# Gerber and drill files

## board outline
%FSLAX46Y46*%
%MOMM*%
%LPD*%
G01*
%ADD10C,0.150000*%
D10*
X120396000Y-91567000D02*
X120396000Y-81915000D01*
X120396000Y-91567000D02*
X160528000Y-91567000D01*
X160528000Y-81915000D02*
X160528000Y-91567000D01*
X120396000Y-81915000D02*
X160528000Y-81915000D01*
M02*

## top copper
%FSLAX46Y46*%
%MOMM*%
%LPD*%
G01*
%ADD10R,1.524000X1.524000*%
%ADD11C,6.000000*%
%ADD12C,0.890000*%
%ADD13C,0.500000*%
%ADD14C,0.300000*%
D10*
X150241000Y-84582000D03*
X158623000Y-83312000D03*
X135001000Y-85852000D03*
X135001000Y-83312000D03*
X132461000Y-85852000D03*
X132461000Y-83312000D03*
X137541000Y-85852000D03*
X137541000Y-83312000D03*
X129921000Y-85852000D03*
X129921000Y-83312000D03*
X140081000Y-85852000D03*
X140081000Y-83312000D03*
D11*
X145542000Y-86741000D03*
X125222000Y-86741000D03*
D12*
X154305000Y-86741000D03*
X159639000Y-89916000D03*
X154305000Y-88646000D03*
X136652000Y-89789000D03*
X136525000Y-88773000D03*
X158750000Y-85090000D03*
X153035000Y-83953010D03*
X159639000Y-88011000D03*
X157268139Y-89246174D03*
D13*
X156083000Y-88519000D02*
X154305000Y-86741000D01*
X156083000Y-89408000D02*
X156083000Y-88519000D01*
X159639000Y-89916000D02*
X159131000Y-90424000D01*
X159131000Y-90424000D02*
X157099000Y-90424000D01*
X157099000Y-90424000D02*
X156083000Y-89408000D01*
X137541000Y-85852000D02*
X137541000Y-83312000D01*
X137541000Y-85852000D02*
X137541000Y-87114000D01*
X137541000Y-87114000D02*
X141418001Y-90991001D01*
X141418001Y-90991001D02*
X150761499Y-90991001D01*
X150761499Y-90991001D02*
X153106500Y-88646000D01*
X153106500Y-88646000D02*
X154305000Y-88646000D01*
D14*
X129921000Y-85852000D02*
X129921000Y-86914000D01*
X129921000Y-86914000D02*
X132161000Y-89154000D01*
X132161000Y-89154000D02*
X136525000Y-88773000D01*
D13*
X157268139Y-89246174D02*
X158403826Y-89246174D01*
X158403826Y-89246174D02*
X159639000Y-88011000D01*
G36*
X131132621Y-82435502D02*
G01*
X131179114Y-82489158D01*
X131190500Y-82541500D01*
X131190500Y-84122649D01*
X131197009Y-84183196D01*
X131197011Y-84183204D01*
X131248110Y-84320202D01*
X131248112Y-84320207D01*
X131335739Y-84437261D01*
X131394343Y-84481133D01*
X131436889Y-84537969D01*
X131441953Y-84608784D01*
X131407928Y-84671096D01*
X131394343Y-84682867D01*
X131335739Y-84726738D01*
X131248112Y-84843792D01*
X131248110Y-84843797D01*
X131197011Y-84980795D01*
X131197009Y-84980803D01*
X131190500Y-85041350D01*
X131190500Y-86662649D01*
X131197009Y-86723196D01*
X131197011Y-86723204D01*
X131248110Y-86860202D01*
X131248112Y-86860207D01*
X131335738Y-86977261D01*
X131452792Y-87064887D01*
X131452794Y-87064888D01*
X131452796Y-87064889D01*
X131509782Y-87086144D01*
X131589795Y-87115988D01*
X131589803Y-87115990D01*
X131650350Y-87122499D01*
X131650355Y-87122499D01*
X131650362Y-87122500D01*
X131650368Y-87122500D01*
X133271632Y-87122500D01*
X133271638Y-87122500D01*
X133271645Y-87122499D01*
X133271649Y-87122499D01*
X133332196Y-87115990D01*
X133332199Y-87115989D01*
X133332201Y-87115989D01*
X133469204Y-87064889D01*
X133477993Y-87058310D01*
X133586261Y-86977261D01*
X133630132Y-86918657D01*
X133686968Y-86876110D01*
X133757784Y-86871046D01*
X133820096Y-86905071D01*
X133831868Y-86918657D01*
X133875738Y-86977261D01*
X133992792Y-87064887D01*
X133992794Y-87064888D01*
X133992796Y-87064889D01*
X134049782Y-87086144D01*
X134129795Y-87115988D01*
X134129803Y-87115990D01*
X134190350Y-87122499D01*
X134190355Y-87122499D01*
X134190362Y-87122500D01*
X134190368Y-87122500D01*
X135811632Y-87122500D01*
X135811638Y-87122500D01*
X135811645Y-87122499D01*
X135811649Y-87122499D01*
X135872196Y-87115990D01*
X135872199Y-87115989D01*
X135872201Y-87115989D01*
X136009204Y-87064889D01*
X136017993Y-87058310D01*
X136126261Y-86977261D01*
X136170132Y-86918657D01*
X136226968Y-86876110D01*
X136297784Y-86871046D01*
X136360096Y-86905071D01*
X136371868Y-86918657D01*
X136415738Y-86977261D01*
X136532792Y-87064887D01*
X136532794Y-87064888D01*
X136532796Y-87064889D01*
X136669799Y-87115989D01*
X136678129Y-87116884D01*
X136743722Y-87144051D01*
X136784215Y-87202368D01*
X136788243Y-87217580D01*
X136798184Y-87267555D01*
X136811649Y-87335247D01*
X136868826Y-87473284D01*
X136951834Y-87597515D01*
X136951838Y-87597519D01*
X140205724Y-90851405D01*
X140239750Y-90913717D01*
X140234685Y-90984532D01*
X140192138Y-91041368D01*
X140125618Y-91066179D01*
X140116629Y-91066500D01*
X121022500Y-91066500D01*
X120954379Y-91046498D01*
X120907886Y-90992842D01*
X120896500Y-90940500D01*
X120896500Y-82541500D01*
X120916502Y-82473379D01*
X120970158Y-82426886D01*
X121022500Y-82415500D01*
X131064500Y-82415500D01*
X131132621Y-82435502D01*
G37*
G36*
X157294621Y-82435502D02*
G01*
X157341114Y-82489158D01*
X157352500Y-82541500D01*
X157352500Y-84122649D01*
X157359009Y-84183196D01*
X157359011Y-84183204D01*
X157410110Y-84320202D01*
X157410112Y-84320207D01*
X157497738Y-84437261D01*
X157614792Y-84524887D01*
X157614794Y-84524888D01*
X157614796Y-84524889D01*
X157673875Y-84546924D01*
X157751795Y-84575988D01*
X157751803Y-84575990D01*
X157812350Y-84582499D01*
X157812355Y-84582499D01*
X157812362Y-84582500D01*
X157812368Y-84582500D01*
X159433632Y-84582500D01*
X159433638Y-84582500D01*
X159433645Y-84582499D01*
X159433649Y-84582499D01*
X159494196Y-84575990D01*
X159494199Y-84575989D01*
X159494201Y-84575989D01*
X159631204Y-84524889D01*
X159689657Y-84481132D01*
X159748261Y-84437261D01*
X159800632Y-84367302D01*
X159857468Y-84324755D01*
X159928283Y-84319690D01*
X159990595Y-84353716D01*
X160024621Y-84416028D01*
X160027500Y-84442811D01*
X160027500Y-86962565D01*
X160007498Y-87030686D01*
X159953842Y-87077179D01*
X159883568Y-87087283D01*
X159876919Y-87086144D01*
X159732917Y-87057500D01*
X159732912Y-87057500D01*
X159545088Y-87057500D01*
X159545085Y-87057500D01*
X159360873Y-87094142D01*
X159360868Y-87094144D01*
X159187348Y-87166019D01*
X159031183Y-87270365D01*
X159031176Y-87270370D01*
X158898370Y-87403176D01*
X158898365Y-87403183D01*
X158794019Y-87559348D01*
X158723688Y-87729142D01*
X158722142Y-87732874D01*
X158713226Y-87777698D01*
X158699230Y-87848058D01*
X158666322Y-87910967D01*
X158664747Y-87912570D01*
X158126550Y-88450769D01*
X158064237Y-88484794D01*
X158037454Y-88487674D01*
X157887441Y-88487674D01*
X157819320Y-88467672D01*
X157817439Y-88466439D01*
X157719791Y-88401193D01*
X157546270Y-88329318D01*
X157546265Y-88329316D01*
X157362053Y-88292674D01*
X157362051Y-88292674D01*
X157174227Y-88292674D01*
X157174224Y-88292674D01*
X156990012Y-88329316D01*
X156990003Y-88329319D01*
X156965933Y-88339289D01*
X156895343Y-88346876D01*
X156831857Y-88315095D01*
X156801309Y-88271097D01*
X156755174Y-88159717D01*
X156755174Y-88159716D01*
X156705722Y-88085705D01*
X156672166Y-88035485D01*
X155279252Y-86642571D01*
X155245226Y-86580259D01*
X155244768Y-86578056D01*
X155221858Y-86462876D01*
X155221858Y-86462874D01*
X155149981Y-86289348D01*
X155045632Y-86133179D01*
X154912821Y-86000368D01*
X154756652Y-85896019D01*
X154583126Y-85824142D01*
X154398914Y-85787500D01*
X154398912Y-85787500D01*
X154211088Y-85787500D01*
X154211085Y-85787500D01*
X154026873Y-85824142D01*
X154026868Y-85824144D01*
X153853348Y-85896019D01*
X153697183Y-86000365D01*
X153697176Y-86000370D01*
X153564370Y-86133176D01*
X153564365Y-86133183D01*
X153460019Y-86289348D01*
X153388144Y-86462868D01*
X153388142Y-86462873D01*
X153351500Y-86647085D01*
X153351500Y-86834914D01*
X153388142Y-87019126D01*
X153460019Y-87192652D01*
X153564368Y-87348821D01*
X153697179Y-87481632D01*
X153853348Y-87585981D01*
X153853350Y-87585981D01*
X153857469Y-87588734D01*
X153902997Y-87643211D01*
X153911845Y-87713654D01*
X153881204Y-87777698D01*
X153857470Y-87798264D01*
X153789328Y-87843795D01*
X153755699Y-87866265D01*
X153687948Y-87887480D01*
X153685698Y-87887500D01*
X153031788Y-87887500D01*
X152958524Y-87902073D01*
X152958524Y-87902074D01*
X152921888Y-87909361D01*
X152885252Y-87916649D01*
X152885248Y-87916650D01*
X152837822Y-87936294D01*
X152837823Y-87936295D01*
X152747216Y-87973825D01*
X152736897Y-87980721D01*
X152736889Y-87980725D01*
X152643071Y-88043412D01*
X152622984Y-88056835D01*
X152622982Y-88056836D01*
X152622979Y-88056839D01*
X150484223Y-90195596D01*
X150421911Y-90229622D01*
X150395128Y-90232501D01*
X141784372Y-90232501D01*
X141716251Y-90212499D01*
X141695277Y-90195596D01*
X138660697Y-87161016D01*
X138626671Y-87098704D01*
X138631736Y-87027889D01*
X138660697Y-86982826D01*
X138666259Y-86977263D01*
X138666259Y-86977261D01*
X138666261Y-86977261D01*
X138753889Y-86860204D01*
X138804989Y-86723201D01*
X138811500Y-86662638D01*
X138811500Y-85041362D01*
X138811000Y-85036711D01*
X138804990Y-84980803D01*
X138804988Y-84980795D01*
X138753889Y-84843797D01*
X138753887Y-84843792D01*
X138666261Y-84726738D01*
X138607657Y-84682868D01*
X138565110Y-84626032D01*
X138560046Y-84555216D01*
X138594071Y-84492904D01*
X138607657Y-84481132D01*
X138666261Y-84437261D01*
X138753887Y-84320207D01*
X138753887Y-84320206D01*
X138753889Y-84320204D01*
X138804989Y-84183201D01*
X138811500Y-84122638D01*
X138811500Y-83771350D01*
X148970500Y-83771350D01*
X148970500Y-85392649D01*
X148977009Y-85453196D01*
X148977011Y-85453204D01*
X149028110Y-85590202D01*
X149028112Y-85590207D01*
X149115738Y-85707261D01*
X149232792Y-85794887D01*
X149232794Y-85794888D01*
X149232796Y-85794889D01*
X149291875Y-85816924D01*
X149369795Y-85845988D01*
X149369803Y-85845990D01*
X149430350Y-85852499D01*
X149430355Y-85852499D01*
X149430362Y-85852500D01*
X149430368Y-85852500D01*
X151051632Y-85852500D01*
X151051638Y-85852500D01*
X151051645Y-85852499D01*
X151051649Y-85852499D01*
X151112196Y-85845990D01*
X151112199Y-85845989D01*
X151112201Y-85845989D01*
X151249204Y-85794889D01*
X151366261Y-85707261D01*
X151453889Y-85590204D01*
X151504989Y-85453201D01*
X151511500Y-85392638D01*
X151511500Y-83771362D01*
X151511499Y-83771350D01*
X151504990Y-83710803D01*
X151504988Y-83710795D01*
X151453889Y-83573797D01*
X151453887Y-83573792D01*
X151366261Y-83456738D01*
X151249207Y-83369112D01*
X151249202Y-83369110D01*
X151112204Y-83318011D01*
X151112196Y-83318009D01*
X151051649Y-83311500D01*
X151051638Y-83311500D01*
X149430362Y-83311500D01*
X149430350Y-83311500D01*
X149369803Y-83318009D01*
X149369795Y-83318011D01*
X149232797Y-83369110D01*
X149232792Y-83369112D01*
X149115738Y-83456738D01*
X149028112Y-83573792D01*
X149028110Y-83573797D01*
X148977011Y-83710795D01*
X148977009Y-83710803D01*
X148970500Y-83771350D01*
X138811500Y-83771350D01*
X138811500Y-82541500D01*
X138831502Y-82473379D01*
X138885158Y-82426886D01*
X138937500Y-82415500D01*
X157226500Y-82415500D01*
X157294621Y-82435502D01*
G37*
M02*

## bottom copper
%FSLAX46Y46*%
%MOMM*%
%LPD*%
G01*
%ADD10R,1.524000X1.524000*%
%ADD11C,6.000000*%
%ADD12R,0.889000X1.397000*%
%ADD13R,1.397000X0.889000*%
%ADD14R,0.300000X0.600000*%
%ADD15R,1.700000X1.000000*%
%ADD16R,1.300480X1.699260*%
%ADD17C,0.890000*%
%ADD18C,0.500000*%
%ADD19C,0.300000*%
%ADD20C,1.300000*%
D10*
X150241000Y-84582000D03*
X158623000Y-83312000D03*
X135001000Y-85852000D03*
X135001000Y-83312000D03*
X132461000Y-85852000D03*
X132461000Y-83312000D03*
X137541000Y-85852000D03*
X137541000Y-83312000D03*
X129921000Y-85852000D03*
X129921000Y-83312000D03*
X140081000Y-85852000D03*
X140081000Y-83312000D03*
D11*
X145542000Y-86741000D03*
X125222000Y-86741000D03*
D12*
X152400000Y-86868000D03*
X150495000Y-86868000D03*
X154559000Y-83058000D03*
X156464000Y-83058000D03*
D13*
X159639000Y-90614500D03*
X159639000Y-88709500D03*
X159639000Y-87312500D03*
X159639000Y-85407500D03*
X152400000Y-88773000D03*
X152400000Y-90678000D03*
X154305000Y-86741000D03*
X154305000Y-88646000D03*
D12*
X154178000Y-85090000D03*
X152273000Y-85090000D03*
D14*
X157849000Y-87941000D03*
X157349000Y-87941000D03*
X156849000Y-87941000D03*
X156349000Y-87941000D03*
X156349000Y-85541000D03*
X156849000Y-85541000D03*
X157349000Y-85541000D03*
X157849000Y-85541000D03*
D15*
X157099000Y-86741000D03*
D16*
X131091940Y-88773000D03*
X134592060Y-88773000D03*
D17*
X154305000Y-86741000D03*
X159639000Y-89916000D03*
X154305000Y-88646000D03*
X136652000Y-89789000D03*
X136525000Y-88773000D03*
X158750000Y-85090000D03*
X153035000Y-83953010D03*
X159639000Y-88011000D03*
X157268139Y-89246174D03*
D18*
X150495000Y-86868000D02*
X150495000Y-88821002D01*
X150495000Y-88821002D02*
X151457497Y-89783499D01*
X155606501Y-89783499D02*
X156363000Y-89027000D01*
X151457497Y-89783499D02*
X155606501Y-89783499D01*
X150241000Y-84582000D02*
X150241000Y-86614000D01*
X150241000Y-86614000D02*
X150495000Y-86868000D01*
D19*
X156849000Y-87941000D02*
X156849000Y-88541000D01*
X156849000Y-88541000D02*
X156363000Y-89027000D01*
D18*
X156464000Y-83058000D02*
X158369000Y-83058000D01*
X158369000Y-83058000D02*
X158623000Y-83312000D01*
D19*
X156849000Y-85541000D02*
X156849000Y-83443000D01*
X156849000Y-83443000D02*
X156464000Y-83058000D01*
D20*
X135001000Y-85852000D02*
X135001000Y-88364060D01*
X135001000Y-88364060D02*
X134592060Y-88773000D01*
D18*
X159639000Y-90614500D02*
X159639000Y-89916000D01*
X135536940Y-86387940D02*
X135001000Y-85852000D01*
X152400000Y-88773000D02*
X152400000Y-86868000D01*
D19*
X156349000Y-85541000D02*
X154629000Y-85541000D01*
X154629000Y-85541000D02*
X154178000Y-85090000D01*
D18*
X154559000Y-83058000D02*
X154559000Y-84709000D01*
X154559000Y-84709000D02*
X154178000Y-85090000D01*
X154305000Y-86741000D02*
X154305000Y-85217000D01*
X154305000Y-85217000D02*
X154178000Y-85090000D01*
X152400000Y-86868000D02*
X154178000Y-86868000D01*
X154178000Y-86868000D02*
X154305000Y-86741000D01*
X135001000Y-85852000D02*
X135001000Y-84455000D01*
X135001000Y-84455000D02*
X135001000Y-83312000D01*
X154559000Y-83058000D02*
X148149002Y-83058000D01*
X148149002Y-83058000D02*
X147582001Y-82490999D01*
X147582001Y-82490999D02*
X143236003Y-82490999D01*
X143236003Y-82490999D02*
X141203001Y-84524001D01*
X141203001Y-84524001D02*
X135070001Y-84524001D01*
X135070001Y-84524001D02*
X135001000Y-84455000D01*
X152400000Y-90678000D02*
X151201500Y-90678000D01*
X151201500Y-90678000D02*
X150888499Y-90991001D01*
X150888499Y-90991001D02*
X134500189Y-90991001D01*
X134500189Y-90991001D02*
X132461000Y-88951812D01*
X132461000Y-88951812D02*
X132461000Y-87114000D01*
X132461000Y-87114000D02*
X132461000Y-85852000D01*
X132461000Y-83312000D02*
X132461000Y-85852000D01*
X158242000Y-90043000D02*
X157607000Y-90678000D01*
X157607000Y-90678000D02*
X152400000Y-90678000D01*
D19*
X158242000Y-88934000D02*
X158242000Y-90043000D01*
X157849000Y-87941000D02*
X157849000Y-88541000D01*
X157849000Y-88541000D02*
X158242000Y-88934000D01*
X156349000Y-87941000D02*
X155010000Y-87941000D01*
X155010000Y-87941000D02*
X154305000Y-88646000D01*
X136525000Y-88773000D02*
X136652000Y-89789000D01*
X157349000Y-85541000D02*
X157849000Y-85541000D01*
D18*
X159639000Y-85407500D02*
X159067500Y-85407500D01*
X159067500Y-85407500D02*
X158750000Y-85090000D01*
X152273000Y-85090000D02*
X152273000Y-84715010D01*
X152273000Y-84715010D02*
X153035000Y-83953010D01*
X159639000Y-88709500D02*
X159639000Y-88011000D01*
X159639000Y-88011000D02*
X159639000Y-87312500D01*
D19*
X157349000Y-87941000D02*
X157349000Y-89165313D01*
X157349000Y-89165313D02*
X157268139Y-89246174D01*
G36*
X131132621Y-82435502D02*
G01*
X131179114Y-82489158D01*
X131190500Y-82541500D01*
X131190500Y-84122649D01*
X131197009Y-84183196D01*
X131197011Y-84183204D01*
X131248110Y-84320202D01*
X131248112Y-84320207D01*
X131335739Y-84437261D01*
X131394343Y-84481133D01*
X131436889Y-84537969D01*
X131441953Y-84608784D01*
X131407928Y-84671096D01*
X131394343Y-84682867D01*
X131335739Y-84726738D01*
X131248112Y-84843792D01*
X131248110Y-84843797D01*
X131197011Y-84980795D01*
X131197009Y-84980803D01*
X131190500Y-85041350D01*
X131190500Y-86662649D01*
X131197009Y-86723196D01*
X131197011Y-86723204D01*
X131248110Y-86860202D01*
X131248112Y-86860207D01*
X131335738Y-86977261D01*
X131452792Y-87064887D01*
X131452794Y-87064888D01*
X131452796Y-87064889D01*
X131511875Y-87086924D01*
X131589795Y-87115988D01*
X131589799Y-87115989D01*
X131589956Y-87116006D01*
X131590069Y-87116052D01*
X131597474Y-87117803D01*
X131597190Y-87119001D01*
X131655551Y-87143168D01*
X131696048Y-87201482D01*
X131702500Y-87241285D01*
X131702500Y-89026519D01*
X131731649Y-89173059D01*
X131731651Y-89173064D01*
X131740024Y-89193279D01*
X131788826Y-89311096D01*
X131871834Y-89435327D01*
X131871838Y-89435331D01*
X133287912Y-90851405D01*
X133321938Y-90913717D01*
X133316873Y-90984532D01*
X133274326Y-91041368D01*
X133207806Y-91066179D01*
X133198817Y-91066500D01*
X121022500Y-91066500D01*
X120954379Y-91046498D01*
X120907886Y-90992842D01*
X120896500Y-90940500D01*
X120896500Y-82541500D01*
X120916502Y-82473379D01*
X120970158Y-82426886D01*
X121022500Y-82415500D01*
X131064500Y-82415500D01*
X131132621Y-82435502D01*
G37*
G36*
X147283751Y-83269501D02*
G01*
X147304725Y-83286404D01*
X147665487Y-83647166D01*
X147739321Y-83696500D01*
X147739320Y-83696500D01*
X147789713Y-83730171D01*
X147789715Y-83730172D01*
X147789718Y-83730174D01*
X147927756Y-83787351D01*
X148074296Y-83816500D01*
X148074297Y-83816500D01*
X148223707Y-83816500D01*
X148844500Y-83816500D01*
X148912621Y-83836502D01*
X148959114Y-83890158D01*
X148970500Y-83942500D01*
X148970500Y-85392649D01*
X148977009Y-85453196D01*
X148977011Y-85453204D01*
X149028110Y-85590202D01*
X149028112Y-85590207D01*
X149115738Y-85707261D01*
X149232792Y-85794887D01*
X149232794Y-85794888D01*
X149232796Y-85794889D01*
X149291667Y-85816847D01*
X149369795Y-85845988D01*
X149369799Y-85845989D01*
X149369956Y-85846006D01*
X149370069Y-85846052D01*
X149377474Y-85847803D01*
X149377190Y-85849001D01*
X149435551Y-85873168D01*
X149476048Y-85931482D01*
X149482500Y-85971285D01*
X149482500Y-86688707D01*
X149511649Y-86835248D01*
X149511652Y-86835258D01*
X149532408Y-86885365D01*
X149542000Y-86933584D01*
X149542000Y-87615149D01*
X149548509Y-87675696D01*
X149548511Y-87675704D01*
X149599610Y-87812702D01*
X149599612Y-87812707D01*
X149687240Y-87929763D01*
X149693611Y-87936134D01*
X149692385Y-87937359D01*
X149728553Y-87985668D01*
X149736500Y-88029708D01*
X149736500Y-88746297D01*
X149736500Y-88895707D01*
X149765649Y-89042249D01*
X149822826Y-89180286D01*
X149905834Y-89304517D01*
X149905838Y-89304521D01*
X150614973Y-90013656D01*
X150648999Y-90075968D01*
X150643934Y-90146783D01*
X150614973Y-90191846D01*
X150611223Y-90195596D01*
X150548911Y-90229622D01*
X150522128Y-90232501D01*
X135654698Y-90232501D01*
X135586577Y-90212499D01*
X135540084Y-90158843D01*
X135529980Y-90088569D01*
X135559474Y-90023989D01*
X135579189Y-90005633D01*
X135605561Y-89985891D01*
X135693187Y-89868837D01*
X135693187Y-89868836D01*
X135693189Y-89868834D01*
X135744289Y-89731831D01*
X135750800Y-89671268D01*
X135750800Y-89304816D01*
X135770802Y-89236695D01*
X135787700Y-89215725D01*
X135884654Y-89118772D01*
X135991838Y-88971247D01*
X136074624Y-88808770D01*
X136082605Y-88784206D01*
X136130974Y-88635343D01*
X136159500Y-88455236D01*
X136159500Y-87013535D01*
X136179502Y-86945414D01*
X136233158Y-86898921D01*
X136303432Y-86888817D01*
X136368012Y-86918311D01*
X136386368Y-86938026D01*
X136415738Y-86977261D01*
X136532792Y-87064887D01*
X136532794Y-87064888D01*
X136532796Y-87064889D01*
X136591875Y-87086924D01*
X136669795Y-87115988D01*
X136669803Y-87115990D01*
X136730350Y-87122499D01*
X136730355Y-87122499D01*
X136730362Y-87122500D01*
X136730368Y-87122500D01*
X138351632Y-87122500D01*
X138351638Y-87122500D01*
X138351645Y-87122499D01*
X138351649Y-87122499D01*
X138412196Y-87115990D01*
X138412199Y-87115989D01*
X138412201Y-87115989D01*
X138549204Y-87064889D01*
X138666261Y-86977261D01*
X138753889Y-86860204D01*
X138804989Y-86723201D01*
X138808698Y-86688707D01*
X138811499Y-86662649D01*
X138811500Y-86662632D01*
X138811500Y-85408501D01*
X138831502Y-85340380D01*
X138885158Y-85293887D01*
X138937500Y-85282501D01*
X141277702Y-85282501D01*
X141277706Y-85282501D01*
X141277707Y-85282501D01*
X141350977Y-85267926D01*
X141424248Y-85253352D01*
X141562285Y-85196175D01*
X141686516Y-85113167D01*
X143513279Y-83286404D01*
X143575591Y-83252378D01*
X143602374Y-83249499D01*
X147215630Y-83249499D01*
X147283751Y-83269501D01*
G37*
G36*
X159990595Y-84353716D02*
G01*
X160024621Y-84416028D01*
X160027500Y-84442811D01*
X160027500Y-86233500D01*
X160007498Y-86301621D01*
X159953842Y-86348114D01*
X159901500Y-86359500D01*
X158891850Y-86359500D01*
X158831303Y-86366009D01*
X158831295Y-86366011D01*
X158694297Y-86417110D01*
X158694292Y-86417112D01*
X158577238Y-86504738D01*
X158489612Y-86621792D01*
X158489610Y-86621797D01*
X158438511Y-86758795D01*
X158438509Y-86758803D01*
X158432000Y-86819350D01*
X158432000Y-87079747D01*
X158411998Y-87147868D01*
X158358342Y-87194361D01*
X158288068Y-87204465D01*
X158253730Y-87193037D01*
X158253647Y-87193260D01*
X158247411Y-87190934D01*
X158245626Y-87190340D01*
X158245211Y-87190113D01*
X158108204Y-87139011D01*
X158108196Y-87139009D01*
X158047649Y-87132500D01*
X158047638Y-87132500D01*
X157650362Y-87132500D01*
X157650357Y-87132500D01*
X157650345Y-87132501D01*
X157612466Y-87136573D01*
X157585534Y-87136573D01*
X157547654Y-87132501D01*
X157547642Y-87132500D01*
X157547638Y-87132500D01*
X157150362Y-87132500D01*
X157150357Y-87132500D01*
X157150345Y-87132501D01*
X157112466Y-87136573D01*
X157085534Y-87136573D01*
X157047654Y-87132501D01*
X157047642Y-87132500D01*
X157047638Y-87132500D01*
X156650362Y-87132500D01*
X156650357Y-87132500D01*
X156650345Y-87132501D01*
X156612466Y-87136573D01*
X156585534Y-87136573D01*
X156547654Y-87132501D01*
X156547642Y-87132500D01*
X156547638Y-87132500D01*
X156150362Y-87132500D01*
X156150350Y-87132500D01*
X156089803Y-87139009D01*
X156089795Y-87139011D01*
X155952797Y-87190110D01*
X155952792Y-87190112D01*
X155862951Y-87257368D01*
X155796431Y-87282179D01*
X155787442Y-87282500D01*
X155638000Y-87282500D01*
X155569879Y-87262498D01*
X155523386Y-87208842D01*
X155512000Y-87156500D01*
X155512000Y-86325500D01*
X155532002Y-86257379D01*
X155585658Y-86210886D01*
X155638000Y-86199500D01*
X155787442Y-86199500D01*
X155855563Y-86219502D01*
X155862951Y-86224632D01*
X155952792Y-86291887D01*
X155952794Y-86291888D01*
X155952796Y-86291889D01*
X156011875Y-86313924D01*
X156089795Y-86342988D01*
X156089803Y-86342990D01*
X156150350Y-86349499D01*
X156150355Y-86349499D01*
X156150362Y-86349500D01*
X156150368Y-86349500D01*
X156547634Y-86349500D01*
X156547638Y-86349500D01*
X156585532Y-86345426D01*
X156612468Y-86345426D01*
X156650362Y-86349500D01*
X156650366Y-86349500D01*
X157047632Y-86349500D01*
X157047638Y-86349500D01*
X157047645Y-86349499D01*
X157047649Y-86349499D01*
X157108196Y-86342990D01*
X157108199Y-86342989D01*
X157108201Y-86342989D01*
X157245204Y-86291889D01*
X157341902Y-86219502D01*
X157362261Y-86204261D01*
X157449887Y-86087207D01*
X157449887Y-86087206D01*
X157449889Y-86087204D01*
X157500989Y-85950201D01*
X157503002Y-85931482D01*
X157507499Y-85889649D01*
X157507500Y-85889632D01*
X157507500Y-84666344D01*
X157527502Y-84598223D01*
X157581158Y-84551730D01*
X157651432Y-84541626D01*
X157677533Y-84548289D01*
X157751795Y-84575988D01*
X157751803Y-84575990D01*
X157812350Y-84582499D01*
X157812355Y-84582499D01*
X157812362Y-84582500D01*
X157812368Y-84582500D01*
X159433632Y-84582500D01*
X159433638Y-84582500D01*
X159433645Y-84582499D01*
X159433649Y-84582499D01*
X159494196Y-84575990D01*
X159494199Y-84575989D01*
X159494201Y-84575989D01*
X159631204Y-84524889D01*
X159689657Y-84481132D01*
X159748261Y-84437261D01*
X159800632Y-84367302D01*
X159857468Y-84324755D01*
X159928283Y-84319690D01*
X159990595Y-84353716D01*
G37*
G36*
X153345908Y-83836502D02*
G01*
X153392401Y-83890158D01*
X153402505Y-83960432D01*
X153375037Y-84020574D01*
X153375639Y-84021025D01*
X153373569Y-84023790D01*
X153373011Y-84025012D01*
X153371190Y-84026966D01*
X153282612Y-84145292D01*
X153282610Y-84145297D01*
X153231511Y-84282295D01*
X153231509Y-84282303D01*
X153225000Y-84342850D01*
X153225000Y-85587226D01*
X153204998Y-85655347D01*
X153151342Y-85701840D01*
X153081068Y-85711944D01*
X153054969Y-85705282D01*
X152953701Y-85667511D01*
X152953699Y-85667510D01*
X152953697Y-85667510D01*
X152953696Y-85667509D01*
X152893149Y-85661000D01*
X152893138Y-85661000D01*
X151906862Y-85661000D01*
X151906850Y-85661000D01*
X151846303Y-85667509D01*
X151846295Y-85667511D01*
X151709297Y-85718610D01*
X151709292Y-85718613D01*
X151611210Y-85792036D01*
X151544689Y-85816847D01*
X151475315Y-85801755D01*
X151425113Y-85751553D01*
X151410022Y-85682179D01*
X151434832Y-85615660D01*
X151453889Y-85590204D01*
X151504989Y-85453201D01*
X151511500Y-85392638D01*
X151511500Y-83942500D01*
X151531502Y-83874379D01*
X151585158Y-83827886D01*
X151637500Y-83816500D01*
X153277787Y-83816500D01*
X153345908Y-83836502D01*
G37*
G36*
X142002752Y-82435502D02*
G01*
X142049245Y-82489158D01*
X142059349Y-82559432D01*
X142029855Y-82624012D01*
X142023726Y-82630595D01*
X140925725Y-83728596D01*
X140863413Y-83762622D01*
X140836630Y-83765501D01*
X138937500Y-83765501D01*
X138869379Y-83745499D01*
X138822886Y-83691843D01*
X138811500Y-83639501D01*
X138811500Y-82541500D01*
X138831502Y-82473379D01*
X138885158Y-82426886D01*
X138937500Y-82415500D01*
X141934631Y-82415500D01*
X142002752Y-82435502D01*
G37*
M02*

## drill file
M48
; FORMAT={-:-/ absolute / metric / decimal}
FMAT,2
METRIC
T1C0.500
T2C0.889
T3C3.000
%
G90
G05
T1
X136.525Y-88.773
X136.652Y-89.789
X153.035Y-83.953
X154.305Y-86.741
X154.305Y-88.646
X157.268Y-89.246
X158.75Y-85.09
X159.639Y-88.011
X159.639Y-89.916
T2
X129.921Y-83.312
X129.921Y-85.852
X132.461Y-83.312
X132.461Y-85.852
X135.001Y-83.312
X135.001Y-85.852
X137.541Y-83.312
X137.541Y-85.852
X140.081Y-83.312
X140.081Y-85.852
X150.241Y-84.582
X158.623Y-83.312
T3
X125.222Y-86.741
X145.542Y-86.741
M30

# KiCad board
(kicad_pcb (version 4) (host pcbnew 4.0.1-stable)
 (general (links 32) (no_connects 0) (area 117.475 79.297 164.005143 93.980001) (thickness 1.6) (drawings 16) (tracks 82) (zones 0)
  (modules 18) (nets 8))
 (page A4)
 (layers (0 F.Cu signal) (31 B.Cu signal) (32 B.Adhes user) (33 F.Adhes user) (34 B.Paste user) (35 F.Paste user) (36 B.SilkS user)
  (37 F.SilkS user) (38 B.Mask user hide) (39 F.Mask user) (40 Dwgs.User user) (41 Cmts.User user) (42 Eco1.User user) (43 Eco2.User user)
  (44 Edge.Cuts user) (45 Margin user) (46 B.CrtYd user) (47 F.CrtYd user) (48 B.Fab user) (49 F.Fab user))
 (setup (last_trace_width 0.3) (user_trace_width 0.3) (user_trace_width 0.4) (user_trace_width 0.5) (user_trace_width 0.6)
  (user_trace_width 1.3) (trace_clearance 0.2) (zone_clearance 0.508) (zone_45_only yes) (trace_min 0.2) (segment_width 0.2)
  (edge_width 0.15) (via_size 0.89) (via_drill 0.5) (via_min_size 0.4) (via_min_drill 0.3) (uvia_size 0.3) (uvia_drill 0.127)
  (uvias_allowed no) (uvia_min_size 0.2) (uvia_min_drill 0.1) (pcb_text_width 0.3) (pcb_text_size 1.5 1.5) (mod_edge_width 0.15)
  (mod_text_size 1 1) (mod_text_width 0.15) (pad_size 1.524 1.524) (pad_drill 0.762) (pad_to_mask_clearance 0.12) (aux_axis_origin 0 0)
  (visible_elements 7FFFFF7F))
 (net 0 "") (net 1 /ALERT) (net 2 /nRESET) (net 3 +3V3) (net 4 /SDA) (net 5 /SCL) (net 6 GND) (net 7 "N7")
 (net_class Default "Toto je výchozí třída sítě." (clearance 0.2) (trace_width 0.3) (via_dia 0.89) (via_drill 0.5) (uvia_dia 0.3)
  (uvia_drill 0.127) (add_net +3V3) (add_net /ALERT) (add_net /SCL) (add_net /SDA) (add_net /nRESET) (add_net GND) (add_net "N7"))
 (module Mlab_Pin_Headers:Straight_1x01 (layer F.Cu) (at 150.241 84.582)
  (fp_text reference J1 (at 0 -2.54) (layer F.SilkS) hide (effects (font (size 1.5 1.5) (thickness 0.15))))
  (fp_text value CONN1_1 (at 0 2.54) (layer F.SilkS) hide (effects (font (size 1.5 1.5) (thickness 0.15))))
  (pad 1 thru_hole rect (at 0 0) (size 1.524 1.524) (drill 0.889) (layers *.Cu *.Mask F.SilkS) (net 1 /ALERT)))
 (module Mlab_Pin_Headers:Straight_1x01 (layer F.Cu) (at 158.623 83.312)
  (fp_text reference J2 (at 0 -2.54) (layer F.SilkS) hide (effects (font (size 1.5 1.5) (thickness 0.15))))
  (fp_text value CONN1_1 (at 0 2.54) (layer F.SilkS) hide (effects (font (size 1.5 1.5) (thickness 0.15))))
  (pad 1 thru_hole rect (at 0 0) (size 1.524 1.524) (drill 0.889) (layers *.Cu *.Mask F.SilkS) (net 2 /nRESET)))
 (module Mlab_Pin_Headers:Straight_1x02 (layer F.Cu) (at 135.001 84.582)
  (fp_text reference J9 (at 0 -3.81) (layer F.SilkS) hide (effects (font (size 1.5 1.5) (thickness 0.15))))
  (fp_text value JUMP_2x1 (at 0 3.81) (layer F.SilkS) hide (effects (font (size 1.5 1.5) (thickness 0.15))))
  (pad 2 thru_hole rect (at 0 1.27) (size 1.524 1.524) (drill 0.889) (layers *.Cu *.Mask F.SilkS) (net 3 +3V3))
  (pad 1 thru_hole rect (at 0 -1.27) (size 1.524 1.524) (drill 0.889) (layers *.Cu *.Mask F.SilkS) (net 3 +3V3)))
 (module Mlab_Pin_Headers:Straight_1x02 (layer F.Cu) (at 132.461 84.582)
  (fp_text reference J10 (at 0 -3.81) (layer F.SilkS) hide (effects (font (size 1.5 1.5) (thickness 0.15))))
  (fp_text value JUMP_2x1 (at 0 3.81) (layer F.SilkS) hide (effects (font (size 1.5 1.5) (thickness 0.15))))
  (pad 2 thru_hole rect (at 0 1.27) (size 1.524 1.524) (drill 0.889) (layers *.Cu *.Mask F.SilkS) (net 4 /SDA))
  (pad 1 thru_hole rect (at 0 -1.27) (size 1.524 1.524) (drill 0.889) (layers *.Cu *.Mask F.SilkS) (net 4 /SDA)))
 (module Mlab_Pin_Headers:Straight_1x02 (layer F.Cu) (at 137.541 84.582)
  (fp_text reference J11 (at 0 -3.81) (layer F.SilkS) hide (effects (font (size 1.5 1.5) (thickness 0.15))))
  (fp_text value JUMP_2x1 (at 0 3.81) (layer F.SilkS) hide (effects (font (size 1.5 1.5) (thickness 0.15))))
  (pad 2 thru_hole rect (at 0 1.27) (size 1.524 1.524) (drill 0.889) (layers *.Cu *.Mask F.SilkS) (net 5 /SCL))
  (pad 1 thru_hole rect (at 0 -1.27) (size 1.524 1.524) (drill 0.889) (layers *.Cu *.Mask F.SilkS) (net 5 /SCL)))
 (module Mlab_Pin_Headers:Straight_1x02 (layer F.Cu) (at 129.921 84.582)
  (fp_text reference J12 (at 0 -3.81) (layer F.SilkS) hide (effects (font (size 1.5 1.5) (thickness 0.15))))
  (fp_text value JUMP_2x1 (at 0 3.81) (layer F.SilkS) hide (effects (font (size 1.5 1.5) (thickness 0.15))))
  (pad 2 thru_hole rect (at 0 1.27) (size 1.524 1.524) (drill 0.889) (layers *.Cu *.Mask F.SilkS) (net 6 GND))
  (pad 1 thru_hole rect (at 0 -1.27) (size 1.524 1.524) (drill 0.889) (layers *.Cu *.Mask F.SilkS) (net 6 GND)))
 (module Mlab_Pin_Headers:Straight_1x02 (layer F.Cu) (at 140.081 84.582)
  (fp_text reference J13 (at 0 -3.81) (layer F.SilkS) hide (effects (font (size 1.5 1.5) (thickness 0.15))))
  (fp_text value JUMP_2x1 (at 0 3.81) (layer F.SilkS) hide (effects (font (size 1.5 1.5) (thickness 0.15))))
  (pad 2 thru_hole rect (at 0 1.27) (size 1.524 1.524) (drill 0.889) (layers *.Cu *.Mask F.SilkS) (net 6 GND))
  (pad 1 thru_hole rect (at 0 -1.27) (size 1.524 1.524) (drill 0.889) (layers *.Cu *.Mask F.SilkS) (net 6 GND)))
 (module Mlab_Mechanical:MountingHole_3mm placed (layer F.Cu) (at 145.542 86.741)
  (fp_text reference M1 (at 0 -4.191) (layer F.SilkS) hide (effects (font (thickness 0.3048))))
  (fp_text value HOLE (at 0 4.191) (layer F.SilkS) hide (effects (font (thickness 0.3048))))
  (pad 1 thru_hole circle (at 0 0) (size 6 6) (drill 3) (layers *.Cu *.Adhes *.Mask) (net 6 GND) (clearance 1) (zone_connect 2)))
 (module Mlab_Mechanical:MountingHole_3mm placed (layer F.Cu) (at 125.222 86.741)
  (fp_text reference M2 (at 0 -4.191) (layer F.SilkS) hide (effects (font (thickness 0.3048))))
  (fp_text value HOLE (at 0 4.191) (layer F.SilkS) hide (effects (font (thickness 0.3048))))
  (pad 1 thru_hole circle (at 0 0) (size 6 6) (drill 3) (layers *.Cu *.Adhes *.Mask) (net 6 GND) (clearance 1) (zone_connect 2)))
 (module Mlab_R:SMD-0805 (layer B.Cu) (at 151.4475 86.868 180)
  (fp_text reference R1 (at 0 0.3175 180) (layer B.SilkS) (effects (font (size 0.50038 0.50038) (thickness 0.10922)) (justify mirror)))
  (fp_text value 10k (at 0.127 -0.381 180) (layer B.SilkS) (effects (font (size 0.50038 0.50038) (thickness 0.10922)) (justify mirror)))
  (pad 1 smd rect (at -0.9525 0 180) (size 0.889 1.397) (layers B.Cu B.Paste B.Mask) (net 3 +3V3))
  (pad 2 smd rect (at 0.9525 0 180) (size 0.889 1.397) (layers B.Cu B.Paste B.Mask) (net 1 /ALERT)))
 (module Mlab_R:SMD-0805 (layer B.Cu) (at 155.5115 83.058)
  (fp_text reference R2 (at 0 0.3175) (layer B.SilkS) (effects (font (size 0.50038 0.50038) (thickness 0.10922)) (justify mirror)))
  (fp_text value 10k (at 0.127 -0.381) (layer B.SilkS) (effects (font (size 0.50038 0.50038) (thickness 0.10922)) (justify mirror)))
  (pad 1 smd rect (at -0.9525 0) (size 0.889 1.397) (layers B.Cu B.Paste B.Mask) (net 3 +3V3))
  (pad 2 smd rect (at 0.9525 0) (size 0.889 1.397) (layers B.Cu B.Paste B.Mask) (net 2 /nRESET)))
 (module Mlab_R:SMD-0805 (layer B.Cu) (at 159.639 89.662 90)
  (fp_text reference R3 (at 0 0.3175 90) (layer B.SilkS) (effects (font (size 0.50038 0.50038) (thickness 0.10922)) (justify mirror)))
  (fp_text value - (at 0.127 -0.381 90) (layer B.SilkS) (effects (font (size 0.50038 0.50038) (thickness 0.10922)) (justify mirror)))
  (pad 1 smd rect (at -0.9525 0 90) (size 0.889 1.397) (layers B.Cu B.Paste B.Mask) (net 3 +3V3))
  (pad 2 smd rect (at 0.9525 0 90) (size 0.889 1.397) (layers B.Cu B.Paste B.Mask) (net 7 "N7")))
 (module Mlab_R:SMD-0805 (layer B.Cu) (at 159.639 86.36 90)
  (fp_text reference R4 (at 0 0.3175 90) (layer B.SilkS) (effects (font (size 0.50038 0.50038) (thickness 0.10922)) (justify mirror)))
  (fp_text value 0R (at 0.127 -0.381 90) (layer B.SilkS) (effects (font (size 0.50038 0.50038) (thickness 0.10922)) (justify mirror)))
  (pad 1 smd rect (at -0.9525 0 90) (size 0.889 1.397) (layers B.Cu B.Paste B.Mask) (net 7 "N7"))
  (pad 2 smd rect (at 0.9525 0 90) (size 0.889 1.397) (layers B.Cu B.Paste B.Mask) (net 6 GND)))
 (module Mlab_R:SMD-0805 (layer B.Cu) (at 152.4 89.7255 270)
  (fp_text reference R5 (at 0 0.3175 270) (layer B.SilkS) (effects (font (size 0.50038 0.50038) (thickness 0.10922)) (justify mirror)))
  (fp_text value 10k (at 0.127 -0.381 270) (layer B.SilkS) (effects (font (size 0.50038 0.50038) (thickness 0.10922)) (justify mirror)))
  (pad 1 smd rect (at -0.9525 0 270) (size 0.889 1.397) (layers B.Cu B.Paste B.Mask) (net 3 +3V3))
  (pad 2 smd rect (at 0.9525 0 270) (size 0.889 1.397) (layers B.Cu B.Paste B.Mask) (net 4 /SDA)))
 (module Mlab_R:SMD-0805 (layer B.Cu) (at 154.305 87.6935 270)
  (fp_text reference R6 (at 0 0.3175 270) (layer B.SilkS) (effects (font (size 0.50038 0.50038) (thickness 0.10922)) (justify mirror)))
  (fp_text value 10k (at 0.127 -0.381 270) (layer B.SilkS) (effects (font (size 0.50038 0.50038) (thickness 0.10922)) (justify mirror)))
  (pad 1 smd rect (at -0.9525 0 270) (size 0.889 1.397) (layers B.Cu B.Paste B.Mask) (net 3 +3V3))
  (pad 2 smd rect (at 0.9525 0 270) (size 0.889 1.397) (layers B.Cu B.Paste B.Mask) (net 5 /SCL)))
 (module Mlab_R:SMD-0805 (layer B.Cu) (at 153.2255 85.09 180)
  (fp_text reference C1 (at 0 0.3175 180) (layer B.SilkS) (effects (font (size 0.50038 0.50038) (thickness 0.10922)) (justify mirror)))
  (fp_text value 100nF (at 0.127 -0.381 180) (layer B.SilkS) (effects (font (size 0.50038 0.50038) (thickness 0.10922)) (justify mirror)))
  (pad 1 smd rect (at -0.9525 0 180) (size 0.889 1.397) (layers B.Cu B.Paste B.Mask) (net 3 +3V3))
  (pad 2 smd rect (at 0.9525 0 180) (size 0.889 1.397) (layers B.Cu B.Paste B.Mask) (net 6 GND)))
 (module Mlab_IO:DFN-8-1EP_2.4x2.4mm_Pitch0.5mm (layer B.Cu) (at 157.099 86.741 90)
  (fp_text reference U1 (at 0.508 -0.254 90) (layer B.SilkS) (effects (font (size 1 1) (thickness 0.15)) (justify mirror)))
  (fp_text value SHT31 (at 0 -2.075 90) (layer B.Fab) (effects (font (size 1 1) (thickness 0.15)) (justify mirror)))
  (pad 1 smd rect (at -1.2 0.75 90) (size 0.6 0.3) (layers B.Cu B.Paste B.Mask) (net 4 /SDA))
  (pad 2 smd rect (at -1.2 0.25 90) (size 0.6 0.3) (layers B.Cu B.Paste B.Mask) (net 7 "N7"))
  (pad 3 smd rect (at -1.2 -0.25 90) (size 0.6 0.3) (layers B.Cu B.Paste B.Mask) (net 1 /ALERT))
  (pad 4 smd rect (at -1.2 -0.75 90) (size 0.6 0.3) (layers B.Cu B.Paste B.Mask) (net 5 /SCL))
  (pad 5 smd rect (at 1.2 -0.75 90) (size 0.6 0.3) (layers B.Cu B.Paste B.Mask) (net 3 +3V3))
  (pad 6 smd rect (at 1.2 -0.25 90) (size 0.6 0.3) (layers B.Cu B.Paste B.Mask) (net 2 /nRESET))
  (pad 7 smd rect (at 1.2 0.25 90) (size 0.6 0.3) (layers B.Cu B.Paste B.Mask) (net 6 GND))
  (pad 8 smd rect (at 1.2 0.75 90) (size 0.6 0.3) (layers B.Cu B.Paste B.Mask) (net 6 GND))
  (pad 9 smd rect (at 0 0 90) (size 1 1.7) (layers B.Cu B.Paste B.Mask) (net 6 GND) (solder_paste_margin_ratio -0.2)))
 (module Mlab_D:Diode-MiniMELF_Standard (layer B.Cu) (at 132.842 88.773)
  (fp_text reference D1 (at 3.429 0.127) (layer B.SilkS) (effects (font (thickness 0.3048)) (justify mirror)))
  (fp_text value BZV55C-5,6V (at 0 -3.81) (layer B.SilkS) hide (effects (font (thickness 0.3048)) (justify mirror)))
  (pad 1 smd rect (at -1.75006 0) (size 1.30048 1.69926) (layers B.Cu B.Paste B.Mask) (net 6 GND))
  (pad 2 smd rect (at 1.75006 0) (size 1.30048 1.69926) (layers B.Cu B.Paste B.Mask) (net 3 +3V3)))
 (gr_line (start 120.396 91.567) (end 120.396 81.915) (angle 90) (layer Edge.Cuts) (width 0.15))
 (gr_line (start 120.396 91.567) (end 160.528 91.567) (angle 90) (layer Edge.Cuts) (width 0.15))
 (gr_line (start 160.528 81.915) (end 160.528 91.567) (angle 90) (layer Edge.Cuts) (width 0.15))
 (gr_line (start 120.396 81.915) (end 160.528 81.915) (angle 90) (layer Edge.Cuts) (width 0.15))
 (segment (start 150.495 86.868) (end 150.495 88.821002) (width 0.5) (layer B.Cu) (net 1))
 (segment (start 150.495 88.821002) (end 151.457497 89.783499) (width 0.5) (layer B.Cu) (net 1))
 (segment (start 155.606501 89.783499) (end 156.363 89.027) (width 0.5) (layer B.Cu) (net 1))
 (segment (start 151.457497 89.783499) (end 155.606501 89.783499) (width 0.5) (layer B.Cu) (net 1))
 (segment (start 150.241 84.582) (end 150.241 86.614) (width 0.5) (layer B.Cu) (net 1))
 (segment (start 150.241 86.614) (end 150.495 86.868) (width 0.5) (layer B.Cu) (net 1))
 (segment (start 156.849 87.941) (end 156.849 88.541) (width 0.3) (layer B.Cu) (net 1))
 (segment (start 156.849 88.541) (end 156.363 89.027) (width 0.3) (layer B.Cu) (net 1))
 (segment (start 156.464 83.058) (end 158.369 83.058) (width 0.5) (layer B.Cu) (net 2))
 (segment (start 158.369 83.058) (end 158.623 83.312) (width 0.5) (layer B.Cu) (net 2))
 (segment (start 156.849 85.541) (end 156.849 83.443) (width 0.3) (layer B.Cu) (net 2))
 (segment (start 156.849 83.443) (end 156.464 83.058) (width 0.3) (layer B.Cu) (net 2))
 (segment (start 135.001 85.852) (end 135.001 88.36406) (width 1.3) (layer B.Cu) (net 3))
 (segment (start 135.001 88.36406) (end 134.59206 88.773) (width 1.3) (layer B.Cu) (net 3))
 (segment (start 156.083 88.519) (end 154.305 86.741) (width 0.5) (layer F.Cu) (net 3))
 (segment (start 156.083 89.408) (end 156.083 88.519) (width 0.5) (layer F.Cu) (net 3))
 (segment (start 159.639 89.916) (end 159.131 90.424) (width 0.5) (layer F.Cu) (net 3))
 (segment (start 159.131 90.424) (end 157.099 90.424) (width 0.5) (layer F.Cu) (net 3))
 (segment (start 157.099 90.424) (end 156.083 89.408) (width 0.5) (layer F.Cu) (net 3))
 (via (at 154.305 86.741) (size 0.89) (drill 0.5) (layers F.Cu B.Cu) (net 3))
 (segment (start 159.639 90.6145) (end 159.639 89.916) (width 0.5) (layer B.Cu) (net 3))
 (via (at 159.639 89.916) (size 0.89) (drill 0.5) (layers F.Cu B.Cu) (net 3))
 (segment (start 135.53694 86.38794) (end 135.001 85.852) (width 0.5) (layer B.Cu) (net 3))
 (segment (start 152.4 88.773) (end 152.4 86.868) (width 0.5) (layer B.Cu) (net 3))
 (segment (start 156.349 85.541) (end 154.629 85.541) (width 0.3) (layer B.Cu) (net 3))
 (segment (start 154.629 85.541) (end 154.178 85.09) (width 0.3) (layer B.Cu) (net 3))
 (segment (start 154.559 83.058) (end 154.559 84.709) (width 0.5) (layer B.Cu) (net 3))
 (segment (start 154.559 84.709) (end 154.178 85.09) (width 0.5) (layer B.Cu) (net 3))
 (segment (start 154.305 86.741) (end 154.305 85.217) (width 0.5) (layer B.Cu) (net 3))
 (segment (start 154.305 85.217) (end 154.178 85.09) (width 0.5) (layer B.Cu) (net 3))
 (segment (start 152.4 86.868) (end 154.178 86.868) (width 0.5) (layer B.Cu) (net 3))
 (segment (start 154.178 86.868) (end 154.305 86.741) (width 0.5) (layer B.Cu) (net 3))
 (segment (start 135.001 85.852) (end 135.001 84.455) (width 0.5) (layer B.Cu) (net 3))
 (segment (start 135.001 84.455) (end 135.001 83.312) (width 0.5) (layer B.Cu) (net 3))
 (segment (start 154.559 83.058) (end 148.149002 83.058) (width 0.5) (layer B.Cu) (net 3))
 (segment (start 148.149002 83.058) (end 147.582001 82.490999) (width 0.5) (layer B.Cu) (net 3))
 (segment (start 147.582001 82.490999) (end 143.236003 82.490999) (width 0.5) (layer B.Cu) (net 3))
 (segment (start 143.236003 82.490999) (end 141.203001 84.524001) (width 0.5) (layer B.Cu) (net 3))
 (segment (start 141.203001 84.524001) (end 135.070001 84.524001) (width 0.5) (layer B.Cu) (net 3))
 (segment (start 135.070001 84.524001) (end 135.001 84.455) (width 0.5) (layer B.Cu) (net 3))
 (segment (start 152.4 90.678) (end 151.2015 90.678) (width 0.5) (layer B.Cu) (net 4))
 (segment (start 151.2015 90.678) (end 150.888499 90.991001) (width 0.5) (layer B.Cu) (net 4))
 (segment (start 150.888499 90.991001) (end 134.500189 90.991001) (width 0.5) (layer B.Cu) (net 4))
 (segment (start 134.500189 90.991001) (end 132.461 88.951812) (width 0.5) (layer B.Cu) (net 4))
 (segment (start 132.461 88.951812) (end 132.461 87.114) (width 0.5) (layer B.Cu) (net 4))
 (segment (start 132.461 87.114) (end 132.461 85.852) (width 0.5) (layer B.Cu) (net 4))
 (segment (start 132.461 83.312) (end 132.461 85.852) (width 0.5) (layer B.Cu) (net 4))
 (segment (start 158.242 90.043) (end 157.607 90.678) (width 0.5) (layer B.Cu) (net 4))
 (segment (start 157.607 90.678) (end 152.4 90.678) (width 0.5) (layer B.Cu) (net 4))
 (segment (start 158.242 88.934) (end 158.242 90.043) (width 0.3) (layer B.Cu) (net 4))
 (segment (start 157.849 87.941) (end 157.849 88.541) (width 0.3) (layer B.Cu) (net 4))
 (segment (start 157.849 88.541) (end 158.242 88.934) (width 0.3) (layer B.Cu) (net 4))
 (segment (start 137.541 85.852) (end 137.541 83.312) (width 0.5) (layer F.Cu) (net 5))
 (segment (start 137.541 85.852) (end 137.541 87.114) (width 0.5) (layer F.Cu) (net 5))
 (segment (start 137.541 87.114) (end 141.418001 90.991001) (width 0.5) (layer F.Cu) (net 5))
 (segment (start 141.418001 90.991001) (end 150.761499 90.991001) (width 0.5) (layer F.Cu) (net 5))
 (segment (start 150.761499 90.991001) (end 153.1065 88.646) (width 0.5) (layer F.Cu) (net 5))
 (segment (start 153.1065 88.646) (end 154.305 88.646) (width 0.5) (layer F.Cu) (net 5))
 (via (at 154.305 88.646) (size 0.89) (drill 0.5) (layers F.Cu B.Cu) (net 5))
 (segment (start 156.349 87.941) (end 155.01 87.941) (width 0.3) (layer B.Cu) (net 5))
 (segment (start 155.01 87.941) (end 154.305 88.646) (width 0.3) (layer B.Cu) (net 5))
 (segment (start 136.525 88.773) (end 136.652 89.789) (width 0.3) (layer B.Cu) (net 6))
 (via (at 136.652 89.789) (size 0.89) (drill 0.5) (layers F.Cu B.Cu) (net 6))
 (segment (start 129.921 85.852) (end 129.921 86.914) (width 0.3) (layer F.Cu) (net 6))
 (segment (start 129.921 86.914) (end 132.161 89.154) (width 0.3) (layer F.Cu) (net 6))
 (segment (start 132.161 89.154) (end 136.525 88.773) (width 0.3) (layer F.Cu) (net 6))
 (via (at 136.525 88.773) (size 0.89) (drill 0.5) (layers F.Cu B.Cu) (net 6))
 (segment (start 157.349 85.541) (end 157.849 85.541) (width 0.3) (layer B.Cu) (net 6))
 (segment (start 159.639 85.4075) (end 159.0675 85.4075) (width 0.5) (layer B.Cu) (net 6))
 (segment (start 159.0675 85.4075) (end 158.75 85.09) (width 0.5) (layer B.Cu) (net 6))
 (via (at 158.75 85.09) (size 0.89) (drill 0.5) (layers F.Cu B.Cu) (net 6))
 (segment (start 152.273 85.09) (end 152.273 84.71501) (width 0.5) (layer B.Cu) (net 6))
 (segment (start 152.273 84.71501) (end 153.035 83.95301) (width 0.5) (layer B.Cu) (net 6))
 (via (at 153.035 83.95301) (size 0.89) (drill 0.5) (layers F.Cu B.Cu) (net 6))
 (segment (start 159.639 88.7095) (end 159.639 88.011) (width 0.5) (layer B.Cu) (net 7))
 (segment (start 159.639 88.011) (end 159.639 87.3125) (width 0.5) (layer B.Cu) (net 7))
 (segment (start 157.268139 89.246174) (end 158.403826 89.246174) (width 0.5) (layer F.Cu) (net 7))
 (segment (start 158.403826 89.246174) (end 159.639 88.011) (width 0.5) (layer F.Cu) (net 7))
 (via (at 159.639 88.011) (size 0.89) (drill 0.5) (layers F.Cu B.Cu) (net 7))
 (segment (start 157.349 87.941) (end 157.349 89.165313) (width 0.3) (layer B.Cu) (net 7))
 (segment (start 157.349 89.165313) (end 157.268139 89.246174) (width 0.3) (layer B.Cu) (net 7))
 (via (at 157.268139 89.246174) (size 0.89) (drill 0.5) (layers F.Cu B.Cu) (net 7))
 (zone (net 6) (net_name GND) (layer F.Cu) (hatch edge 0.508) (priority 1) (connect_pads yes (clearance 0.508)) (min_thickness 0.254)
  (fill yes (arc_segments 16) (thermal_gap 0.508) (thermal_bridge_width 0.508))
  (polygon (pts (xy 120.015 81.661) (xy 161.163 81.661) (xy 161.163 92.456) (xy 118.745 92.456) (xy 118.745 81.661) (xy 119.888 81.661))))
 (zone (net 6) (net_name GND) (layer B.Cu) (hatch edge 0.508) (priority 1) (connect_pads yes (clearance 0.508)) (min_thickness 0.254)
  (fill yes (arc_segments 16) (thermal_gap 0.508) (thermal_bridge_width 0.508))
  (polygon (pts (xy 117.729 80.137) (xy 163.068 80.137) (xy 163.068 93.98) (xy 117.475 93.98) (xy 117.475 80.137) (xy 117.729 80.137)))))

